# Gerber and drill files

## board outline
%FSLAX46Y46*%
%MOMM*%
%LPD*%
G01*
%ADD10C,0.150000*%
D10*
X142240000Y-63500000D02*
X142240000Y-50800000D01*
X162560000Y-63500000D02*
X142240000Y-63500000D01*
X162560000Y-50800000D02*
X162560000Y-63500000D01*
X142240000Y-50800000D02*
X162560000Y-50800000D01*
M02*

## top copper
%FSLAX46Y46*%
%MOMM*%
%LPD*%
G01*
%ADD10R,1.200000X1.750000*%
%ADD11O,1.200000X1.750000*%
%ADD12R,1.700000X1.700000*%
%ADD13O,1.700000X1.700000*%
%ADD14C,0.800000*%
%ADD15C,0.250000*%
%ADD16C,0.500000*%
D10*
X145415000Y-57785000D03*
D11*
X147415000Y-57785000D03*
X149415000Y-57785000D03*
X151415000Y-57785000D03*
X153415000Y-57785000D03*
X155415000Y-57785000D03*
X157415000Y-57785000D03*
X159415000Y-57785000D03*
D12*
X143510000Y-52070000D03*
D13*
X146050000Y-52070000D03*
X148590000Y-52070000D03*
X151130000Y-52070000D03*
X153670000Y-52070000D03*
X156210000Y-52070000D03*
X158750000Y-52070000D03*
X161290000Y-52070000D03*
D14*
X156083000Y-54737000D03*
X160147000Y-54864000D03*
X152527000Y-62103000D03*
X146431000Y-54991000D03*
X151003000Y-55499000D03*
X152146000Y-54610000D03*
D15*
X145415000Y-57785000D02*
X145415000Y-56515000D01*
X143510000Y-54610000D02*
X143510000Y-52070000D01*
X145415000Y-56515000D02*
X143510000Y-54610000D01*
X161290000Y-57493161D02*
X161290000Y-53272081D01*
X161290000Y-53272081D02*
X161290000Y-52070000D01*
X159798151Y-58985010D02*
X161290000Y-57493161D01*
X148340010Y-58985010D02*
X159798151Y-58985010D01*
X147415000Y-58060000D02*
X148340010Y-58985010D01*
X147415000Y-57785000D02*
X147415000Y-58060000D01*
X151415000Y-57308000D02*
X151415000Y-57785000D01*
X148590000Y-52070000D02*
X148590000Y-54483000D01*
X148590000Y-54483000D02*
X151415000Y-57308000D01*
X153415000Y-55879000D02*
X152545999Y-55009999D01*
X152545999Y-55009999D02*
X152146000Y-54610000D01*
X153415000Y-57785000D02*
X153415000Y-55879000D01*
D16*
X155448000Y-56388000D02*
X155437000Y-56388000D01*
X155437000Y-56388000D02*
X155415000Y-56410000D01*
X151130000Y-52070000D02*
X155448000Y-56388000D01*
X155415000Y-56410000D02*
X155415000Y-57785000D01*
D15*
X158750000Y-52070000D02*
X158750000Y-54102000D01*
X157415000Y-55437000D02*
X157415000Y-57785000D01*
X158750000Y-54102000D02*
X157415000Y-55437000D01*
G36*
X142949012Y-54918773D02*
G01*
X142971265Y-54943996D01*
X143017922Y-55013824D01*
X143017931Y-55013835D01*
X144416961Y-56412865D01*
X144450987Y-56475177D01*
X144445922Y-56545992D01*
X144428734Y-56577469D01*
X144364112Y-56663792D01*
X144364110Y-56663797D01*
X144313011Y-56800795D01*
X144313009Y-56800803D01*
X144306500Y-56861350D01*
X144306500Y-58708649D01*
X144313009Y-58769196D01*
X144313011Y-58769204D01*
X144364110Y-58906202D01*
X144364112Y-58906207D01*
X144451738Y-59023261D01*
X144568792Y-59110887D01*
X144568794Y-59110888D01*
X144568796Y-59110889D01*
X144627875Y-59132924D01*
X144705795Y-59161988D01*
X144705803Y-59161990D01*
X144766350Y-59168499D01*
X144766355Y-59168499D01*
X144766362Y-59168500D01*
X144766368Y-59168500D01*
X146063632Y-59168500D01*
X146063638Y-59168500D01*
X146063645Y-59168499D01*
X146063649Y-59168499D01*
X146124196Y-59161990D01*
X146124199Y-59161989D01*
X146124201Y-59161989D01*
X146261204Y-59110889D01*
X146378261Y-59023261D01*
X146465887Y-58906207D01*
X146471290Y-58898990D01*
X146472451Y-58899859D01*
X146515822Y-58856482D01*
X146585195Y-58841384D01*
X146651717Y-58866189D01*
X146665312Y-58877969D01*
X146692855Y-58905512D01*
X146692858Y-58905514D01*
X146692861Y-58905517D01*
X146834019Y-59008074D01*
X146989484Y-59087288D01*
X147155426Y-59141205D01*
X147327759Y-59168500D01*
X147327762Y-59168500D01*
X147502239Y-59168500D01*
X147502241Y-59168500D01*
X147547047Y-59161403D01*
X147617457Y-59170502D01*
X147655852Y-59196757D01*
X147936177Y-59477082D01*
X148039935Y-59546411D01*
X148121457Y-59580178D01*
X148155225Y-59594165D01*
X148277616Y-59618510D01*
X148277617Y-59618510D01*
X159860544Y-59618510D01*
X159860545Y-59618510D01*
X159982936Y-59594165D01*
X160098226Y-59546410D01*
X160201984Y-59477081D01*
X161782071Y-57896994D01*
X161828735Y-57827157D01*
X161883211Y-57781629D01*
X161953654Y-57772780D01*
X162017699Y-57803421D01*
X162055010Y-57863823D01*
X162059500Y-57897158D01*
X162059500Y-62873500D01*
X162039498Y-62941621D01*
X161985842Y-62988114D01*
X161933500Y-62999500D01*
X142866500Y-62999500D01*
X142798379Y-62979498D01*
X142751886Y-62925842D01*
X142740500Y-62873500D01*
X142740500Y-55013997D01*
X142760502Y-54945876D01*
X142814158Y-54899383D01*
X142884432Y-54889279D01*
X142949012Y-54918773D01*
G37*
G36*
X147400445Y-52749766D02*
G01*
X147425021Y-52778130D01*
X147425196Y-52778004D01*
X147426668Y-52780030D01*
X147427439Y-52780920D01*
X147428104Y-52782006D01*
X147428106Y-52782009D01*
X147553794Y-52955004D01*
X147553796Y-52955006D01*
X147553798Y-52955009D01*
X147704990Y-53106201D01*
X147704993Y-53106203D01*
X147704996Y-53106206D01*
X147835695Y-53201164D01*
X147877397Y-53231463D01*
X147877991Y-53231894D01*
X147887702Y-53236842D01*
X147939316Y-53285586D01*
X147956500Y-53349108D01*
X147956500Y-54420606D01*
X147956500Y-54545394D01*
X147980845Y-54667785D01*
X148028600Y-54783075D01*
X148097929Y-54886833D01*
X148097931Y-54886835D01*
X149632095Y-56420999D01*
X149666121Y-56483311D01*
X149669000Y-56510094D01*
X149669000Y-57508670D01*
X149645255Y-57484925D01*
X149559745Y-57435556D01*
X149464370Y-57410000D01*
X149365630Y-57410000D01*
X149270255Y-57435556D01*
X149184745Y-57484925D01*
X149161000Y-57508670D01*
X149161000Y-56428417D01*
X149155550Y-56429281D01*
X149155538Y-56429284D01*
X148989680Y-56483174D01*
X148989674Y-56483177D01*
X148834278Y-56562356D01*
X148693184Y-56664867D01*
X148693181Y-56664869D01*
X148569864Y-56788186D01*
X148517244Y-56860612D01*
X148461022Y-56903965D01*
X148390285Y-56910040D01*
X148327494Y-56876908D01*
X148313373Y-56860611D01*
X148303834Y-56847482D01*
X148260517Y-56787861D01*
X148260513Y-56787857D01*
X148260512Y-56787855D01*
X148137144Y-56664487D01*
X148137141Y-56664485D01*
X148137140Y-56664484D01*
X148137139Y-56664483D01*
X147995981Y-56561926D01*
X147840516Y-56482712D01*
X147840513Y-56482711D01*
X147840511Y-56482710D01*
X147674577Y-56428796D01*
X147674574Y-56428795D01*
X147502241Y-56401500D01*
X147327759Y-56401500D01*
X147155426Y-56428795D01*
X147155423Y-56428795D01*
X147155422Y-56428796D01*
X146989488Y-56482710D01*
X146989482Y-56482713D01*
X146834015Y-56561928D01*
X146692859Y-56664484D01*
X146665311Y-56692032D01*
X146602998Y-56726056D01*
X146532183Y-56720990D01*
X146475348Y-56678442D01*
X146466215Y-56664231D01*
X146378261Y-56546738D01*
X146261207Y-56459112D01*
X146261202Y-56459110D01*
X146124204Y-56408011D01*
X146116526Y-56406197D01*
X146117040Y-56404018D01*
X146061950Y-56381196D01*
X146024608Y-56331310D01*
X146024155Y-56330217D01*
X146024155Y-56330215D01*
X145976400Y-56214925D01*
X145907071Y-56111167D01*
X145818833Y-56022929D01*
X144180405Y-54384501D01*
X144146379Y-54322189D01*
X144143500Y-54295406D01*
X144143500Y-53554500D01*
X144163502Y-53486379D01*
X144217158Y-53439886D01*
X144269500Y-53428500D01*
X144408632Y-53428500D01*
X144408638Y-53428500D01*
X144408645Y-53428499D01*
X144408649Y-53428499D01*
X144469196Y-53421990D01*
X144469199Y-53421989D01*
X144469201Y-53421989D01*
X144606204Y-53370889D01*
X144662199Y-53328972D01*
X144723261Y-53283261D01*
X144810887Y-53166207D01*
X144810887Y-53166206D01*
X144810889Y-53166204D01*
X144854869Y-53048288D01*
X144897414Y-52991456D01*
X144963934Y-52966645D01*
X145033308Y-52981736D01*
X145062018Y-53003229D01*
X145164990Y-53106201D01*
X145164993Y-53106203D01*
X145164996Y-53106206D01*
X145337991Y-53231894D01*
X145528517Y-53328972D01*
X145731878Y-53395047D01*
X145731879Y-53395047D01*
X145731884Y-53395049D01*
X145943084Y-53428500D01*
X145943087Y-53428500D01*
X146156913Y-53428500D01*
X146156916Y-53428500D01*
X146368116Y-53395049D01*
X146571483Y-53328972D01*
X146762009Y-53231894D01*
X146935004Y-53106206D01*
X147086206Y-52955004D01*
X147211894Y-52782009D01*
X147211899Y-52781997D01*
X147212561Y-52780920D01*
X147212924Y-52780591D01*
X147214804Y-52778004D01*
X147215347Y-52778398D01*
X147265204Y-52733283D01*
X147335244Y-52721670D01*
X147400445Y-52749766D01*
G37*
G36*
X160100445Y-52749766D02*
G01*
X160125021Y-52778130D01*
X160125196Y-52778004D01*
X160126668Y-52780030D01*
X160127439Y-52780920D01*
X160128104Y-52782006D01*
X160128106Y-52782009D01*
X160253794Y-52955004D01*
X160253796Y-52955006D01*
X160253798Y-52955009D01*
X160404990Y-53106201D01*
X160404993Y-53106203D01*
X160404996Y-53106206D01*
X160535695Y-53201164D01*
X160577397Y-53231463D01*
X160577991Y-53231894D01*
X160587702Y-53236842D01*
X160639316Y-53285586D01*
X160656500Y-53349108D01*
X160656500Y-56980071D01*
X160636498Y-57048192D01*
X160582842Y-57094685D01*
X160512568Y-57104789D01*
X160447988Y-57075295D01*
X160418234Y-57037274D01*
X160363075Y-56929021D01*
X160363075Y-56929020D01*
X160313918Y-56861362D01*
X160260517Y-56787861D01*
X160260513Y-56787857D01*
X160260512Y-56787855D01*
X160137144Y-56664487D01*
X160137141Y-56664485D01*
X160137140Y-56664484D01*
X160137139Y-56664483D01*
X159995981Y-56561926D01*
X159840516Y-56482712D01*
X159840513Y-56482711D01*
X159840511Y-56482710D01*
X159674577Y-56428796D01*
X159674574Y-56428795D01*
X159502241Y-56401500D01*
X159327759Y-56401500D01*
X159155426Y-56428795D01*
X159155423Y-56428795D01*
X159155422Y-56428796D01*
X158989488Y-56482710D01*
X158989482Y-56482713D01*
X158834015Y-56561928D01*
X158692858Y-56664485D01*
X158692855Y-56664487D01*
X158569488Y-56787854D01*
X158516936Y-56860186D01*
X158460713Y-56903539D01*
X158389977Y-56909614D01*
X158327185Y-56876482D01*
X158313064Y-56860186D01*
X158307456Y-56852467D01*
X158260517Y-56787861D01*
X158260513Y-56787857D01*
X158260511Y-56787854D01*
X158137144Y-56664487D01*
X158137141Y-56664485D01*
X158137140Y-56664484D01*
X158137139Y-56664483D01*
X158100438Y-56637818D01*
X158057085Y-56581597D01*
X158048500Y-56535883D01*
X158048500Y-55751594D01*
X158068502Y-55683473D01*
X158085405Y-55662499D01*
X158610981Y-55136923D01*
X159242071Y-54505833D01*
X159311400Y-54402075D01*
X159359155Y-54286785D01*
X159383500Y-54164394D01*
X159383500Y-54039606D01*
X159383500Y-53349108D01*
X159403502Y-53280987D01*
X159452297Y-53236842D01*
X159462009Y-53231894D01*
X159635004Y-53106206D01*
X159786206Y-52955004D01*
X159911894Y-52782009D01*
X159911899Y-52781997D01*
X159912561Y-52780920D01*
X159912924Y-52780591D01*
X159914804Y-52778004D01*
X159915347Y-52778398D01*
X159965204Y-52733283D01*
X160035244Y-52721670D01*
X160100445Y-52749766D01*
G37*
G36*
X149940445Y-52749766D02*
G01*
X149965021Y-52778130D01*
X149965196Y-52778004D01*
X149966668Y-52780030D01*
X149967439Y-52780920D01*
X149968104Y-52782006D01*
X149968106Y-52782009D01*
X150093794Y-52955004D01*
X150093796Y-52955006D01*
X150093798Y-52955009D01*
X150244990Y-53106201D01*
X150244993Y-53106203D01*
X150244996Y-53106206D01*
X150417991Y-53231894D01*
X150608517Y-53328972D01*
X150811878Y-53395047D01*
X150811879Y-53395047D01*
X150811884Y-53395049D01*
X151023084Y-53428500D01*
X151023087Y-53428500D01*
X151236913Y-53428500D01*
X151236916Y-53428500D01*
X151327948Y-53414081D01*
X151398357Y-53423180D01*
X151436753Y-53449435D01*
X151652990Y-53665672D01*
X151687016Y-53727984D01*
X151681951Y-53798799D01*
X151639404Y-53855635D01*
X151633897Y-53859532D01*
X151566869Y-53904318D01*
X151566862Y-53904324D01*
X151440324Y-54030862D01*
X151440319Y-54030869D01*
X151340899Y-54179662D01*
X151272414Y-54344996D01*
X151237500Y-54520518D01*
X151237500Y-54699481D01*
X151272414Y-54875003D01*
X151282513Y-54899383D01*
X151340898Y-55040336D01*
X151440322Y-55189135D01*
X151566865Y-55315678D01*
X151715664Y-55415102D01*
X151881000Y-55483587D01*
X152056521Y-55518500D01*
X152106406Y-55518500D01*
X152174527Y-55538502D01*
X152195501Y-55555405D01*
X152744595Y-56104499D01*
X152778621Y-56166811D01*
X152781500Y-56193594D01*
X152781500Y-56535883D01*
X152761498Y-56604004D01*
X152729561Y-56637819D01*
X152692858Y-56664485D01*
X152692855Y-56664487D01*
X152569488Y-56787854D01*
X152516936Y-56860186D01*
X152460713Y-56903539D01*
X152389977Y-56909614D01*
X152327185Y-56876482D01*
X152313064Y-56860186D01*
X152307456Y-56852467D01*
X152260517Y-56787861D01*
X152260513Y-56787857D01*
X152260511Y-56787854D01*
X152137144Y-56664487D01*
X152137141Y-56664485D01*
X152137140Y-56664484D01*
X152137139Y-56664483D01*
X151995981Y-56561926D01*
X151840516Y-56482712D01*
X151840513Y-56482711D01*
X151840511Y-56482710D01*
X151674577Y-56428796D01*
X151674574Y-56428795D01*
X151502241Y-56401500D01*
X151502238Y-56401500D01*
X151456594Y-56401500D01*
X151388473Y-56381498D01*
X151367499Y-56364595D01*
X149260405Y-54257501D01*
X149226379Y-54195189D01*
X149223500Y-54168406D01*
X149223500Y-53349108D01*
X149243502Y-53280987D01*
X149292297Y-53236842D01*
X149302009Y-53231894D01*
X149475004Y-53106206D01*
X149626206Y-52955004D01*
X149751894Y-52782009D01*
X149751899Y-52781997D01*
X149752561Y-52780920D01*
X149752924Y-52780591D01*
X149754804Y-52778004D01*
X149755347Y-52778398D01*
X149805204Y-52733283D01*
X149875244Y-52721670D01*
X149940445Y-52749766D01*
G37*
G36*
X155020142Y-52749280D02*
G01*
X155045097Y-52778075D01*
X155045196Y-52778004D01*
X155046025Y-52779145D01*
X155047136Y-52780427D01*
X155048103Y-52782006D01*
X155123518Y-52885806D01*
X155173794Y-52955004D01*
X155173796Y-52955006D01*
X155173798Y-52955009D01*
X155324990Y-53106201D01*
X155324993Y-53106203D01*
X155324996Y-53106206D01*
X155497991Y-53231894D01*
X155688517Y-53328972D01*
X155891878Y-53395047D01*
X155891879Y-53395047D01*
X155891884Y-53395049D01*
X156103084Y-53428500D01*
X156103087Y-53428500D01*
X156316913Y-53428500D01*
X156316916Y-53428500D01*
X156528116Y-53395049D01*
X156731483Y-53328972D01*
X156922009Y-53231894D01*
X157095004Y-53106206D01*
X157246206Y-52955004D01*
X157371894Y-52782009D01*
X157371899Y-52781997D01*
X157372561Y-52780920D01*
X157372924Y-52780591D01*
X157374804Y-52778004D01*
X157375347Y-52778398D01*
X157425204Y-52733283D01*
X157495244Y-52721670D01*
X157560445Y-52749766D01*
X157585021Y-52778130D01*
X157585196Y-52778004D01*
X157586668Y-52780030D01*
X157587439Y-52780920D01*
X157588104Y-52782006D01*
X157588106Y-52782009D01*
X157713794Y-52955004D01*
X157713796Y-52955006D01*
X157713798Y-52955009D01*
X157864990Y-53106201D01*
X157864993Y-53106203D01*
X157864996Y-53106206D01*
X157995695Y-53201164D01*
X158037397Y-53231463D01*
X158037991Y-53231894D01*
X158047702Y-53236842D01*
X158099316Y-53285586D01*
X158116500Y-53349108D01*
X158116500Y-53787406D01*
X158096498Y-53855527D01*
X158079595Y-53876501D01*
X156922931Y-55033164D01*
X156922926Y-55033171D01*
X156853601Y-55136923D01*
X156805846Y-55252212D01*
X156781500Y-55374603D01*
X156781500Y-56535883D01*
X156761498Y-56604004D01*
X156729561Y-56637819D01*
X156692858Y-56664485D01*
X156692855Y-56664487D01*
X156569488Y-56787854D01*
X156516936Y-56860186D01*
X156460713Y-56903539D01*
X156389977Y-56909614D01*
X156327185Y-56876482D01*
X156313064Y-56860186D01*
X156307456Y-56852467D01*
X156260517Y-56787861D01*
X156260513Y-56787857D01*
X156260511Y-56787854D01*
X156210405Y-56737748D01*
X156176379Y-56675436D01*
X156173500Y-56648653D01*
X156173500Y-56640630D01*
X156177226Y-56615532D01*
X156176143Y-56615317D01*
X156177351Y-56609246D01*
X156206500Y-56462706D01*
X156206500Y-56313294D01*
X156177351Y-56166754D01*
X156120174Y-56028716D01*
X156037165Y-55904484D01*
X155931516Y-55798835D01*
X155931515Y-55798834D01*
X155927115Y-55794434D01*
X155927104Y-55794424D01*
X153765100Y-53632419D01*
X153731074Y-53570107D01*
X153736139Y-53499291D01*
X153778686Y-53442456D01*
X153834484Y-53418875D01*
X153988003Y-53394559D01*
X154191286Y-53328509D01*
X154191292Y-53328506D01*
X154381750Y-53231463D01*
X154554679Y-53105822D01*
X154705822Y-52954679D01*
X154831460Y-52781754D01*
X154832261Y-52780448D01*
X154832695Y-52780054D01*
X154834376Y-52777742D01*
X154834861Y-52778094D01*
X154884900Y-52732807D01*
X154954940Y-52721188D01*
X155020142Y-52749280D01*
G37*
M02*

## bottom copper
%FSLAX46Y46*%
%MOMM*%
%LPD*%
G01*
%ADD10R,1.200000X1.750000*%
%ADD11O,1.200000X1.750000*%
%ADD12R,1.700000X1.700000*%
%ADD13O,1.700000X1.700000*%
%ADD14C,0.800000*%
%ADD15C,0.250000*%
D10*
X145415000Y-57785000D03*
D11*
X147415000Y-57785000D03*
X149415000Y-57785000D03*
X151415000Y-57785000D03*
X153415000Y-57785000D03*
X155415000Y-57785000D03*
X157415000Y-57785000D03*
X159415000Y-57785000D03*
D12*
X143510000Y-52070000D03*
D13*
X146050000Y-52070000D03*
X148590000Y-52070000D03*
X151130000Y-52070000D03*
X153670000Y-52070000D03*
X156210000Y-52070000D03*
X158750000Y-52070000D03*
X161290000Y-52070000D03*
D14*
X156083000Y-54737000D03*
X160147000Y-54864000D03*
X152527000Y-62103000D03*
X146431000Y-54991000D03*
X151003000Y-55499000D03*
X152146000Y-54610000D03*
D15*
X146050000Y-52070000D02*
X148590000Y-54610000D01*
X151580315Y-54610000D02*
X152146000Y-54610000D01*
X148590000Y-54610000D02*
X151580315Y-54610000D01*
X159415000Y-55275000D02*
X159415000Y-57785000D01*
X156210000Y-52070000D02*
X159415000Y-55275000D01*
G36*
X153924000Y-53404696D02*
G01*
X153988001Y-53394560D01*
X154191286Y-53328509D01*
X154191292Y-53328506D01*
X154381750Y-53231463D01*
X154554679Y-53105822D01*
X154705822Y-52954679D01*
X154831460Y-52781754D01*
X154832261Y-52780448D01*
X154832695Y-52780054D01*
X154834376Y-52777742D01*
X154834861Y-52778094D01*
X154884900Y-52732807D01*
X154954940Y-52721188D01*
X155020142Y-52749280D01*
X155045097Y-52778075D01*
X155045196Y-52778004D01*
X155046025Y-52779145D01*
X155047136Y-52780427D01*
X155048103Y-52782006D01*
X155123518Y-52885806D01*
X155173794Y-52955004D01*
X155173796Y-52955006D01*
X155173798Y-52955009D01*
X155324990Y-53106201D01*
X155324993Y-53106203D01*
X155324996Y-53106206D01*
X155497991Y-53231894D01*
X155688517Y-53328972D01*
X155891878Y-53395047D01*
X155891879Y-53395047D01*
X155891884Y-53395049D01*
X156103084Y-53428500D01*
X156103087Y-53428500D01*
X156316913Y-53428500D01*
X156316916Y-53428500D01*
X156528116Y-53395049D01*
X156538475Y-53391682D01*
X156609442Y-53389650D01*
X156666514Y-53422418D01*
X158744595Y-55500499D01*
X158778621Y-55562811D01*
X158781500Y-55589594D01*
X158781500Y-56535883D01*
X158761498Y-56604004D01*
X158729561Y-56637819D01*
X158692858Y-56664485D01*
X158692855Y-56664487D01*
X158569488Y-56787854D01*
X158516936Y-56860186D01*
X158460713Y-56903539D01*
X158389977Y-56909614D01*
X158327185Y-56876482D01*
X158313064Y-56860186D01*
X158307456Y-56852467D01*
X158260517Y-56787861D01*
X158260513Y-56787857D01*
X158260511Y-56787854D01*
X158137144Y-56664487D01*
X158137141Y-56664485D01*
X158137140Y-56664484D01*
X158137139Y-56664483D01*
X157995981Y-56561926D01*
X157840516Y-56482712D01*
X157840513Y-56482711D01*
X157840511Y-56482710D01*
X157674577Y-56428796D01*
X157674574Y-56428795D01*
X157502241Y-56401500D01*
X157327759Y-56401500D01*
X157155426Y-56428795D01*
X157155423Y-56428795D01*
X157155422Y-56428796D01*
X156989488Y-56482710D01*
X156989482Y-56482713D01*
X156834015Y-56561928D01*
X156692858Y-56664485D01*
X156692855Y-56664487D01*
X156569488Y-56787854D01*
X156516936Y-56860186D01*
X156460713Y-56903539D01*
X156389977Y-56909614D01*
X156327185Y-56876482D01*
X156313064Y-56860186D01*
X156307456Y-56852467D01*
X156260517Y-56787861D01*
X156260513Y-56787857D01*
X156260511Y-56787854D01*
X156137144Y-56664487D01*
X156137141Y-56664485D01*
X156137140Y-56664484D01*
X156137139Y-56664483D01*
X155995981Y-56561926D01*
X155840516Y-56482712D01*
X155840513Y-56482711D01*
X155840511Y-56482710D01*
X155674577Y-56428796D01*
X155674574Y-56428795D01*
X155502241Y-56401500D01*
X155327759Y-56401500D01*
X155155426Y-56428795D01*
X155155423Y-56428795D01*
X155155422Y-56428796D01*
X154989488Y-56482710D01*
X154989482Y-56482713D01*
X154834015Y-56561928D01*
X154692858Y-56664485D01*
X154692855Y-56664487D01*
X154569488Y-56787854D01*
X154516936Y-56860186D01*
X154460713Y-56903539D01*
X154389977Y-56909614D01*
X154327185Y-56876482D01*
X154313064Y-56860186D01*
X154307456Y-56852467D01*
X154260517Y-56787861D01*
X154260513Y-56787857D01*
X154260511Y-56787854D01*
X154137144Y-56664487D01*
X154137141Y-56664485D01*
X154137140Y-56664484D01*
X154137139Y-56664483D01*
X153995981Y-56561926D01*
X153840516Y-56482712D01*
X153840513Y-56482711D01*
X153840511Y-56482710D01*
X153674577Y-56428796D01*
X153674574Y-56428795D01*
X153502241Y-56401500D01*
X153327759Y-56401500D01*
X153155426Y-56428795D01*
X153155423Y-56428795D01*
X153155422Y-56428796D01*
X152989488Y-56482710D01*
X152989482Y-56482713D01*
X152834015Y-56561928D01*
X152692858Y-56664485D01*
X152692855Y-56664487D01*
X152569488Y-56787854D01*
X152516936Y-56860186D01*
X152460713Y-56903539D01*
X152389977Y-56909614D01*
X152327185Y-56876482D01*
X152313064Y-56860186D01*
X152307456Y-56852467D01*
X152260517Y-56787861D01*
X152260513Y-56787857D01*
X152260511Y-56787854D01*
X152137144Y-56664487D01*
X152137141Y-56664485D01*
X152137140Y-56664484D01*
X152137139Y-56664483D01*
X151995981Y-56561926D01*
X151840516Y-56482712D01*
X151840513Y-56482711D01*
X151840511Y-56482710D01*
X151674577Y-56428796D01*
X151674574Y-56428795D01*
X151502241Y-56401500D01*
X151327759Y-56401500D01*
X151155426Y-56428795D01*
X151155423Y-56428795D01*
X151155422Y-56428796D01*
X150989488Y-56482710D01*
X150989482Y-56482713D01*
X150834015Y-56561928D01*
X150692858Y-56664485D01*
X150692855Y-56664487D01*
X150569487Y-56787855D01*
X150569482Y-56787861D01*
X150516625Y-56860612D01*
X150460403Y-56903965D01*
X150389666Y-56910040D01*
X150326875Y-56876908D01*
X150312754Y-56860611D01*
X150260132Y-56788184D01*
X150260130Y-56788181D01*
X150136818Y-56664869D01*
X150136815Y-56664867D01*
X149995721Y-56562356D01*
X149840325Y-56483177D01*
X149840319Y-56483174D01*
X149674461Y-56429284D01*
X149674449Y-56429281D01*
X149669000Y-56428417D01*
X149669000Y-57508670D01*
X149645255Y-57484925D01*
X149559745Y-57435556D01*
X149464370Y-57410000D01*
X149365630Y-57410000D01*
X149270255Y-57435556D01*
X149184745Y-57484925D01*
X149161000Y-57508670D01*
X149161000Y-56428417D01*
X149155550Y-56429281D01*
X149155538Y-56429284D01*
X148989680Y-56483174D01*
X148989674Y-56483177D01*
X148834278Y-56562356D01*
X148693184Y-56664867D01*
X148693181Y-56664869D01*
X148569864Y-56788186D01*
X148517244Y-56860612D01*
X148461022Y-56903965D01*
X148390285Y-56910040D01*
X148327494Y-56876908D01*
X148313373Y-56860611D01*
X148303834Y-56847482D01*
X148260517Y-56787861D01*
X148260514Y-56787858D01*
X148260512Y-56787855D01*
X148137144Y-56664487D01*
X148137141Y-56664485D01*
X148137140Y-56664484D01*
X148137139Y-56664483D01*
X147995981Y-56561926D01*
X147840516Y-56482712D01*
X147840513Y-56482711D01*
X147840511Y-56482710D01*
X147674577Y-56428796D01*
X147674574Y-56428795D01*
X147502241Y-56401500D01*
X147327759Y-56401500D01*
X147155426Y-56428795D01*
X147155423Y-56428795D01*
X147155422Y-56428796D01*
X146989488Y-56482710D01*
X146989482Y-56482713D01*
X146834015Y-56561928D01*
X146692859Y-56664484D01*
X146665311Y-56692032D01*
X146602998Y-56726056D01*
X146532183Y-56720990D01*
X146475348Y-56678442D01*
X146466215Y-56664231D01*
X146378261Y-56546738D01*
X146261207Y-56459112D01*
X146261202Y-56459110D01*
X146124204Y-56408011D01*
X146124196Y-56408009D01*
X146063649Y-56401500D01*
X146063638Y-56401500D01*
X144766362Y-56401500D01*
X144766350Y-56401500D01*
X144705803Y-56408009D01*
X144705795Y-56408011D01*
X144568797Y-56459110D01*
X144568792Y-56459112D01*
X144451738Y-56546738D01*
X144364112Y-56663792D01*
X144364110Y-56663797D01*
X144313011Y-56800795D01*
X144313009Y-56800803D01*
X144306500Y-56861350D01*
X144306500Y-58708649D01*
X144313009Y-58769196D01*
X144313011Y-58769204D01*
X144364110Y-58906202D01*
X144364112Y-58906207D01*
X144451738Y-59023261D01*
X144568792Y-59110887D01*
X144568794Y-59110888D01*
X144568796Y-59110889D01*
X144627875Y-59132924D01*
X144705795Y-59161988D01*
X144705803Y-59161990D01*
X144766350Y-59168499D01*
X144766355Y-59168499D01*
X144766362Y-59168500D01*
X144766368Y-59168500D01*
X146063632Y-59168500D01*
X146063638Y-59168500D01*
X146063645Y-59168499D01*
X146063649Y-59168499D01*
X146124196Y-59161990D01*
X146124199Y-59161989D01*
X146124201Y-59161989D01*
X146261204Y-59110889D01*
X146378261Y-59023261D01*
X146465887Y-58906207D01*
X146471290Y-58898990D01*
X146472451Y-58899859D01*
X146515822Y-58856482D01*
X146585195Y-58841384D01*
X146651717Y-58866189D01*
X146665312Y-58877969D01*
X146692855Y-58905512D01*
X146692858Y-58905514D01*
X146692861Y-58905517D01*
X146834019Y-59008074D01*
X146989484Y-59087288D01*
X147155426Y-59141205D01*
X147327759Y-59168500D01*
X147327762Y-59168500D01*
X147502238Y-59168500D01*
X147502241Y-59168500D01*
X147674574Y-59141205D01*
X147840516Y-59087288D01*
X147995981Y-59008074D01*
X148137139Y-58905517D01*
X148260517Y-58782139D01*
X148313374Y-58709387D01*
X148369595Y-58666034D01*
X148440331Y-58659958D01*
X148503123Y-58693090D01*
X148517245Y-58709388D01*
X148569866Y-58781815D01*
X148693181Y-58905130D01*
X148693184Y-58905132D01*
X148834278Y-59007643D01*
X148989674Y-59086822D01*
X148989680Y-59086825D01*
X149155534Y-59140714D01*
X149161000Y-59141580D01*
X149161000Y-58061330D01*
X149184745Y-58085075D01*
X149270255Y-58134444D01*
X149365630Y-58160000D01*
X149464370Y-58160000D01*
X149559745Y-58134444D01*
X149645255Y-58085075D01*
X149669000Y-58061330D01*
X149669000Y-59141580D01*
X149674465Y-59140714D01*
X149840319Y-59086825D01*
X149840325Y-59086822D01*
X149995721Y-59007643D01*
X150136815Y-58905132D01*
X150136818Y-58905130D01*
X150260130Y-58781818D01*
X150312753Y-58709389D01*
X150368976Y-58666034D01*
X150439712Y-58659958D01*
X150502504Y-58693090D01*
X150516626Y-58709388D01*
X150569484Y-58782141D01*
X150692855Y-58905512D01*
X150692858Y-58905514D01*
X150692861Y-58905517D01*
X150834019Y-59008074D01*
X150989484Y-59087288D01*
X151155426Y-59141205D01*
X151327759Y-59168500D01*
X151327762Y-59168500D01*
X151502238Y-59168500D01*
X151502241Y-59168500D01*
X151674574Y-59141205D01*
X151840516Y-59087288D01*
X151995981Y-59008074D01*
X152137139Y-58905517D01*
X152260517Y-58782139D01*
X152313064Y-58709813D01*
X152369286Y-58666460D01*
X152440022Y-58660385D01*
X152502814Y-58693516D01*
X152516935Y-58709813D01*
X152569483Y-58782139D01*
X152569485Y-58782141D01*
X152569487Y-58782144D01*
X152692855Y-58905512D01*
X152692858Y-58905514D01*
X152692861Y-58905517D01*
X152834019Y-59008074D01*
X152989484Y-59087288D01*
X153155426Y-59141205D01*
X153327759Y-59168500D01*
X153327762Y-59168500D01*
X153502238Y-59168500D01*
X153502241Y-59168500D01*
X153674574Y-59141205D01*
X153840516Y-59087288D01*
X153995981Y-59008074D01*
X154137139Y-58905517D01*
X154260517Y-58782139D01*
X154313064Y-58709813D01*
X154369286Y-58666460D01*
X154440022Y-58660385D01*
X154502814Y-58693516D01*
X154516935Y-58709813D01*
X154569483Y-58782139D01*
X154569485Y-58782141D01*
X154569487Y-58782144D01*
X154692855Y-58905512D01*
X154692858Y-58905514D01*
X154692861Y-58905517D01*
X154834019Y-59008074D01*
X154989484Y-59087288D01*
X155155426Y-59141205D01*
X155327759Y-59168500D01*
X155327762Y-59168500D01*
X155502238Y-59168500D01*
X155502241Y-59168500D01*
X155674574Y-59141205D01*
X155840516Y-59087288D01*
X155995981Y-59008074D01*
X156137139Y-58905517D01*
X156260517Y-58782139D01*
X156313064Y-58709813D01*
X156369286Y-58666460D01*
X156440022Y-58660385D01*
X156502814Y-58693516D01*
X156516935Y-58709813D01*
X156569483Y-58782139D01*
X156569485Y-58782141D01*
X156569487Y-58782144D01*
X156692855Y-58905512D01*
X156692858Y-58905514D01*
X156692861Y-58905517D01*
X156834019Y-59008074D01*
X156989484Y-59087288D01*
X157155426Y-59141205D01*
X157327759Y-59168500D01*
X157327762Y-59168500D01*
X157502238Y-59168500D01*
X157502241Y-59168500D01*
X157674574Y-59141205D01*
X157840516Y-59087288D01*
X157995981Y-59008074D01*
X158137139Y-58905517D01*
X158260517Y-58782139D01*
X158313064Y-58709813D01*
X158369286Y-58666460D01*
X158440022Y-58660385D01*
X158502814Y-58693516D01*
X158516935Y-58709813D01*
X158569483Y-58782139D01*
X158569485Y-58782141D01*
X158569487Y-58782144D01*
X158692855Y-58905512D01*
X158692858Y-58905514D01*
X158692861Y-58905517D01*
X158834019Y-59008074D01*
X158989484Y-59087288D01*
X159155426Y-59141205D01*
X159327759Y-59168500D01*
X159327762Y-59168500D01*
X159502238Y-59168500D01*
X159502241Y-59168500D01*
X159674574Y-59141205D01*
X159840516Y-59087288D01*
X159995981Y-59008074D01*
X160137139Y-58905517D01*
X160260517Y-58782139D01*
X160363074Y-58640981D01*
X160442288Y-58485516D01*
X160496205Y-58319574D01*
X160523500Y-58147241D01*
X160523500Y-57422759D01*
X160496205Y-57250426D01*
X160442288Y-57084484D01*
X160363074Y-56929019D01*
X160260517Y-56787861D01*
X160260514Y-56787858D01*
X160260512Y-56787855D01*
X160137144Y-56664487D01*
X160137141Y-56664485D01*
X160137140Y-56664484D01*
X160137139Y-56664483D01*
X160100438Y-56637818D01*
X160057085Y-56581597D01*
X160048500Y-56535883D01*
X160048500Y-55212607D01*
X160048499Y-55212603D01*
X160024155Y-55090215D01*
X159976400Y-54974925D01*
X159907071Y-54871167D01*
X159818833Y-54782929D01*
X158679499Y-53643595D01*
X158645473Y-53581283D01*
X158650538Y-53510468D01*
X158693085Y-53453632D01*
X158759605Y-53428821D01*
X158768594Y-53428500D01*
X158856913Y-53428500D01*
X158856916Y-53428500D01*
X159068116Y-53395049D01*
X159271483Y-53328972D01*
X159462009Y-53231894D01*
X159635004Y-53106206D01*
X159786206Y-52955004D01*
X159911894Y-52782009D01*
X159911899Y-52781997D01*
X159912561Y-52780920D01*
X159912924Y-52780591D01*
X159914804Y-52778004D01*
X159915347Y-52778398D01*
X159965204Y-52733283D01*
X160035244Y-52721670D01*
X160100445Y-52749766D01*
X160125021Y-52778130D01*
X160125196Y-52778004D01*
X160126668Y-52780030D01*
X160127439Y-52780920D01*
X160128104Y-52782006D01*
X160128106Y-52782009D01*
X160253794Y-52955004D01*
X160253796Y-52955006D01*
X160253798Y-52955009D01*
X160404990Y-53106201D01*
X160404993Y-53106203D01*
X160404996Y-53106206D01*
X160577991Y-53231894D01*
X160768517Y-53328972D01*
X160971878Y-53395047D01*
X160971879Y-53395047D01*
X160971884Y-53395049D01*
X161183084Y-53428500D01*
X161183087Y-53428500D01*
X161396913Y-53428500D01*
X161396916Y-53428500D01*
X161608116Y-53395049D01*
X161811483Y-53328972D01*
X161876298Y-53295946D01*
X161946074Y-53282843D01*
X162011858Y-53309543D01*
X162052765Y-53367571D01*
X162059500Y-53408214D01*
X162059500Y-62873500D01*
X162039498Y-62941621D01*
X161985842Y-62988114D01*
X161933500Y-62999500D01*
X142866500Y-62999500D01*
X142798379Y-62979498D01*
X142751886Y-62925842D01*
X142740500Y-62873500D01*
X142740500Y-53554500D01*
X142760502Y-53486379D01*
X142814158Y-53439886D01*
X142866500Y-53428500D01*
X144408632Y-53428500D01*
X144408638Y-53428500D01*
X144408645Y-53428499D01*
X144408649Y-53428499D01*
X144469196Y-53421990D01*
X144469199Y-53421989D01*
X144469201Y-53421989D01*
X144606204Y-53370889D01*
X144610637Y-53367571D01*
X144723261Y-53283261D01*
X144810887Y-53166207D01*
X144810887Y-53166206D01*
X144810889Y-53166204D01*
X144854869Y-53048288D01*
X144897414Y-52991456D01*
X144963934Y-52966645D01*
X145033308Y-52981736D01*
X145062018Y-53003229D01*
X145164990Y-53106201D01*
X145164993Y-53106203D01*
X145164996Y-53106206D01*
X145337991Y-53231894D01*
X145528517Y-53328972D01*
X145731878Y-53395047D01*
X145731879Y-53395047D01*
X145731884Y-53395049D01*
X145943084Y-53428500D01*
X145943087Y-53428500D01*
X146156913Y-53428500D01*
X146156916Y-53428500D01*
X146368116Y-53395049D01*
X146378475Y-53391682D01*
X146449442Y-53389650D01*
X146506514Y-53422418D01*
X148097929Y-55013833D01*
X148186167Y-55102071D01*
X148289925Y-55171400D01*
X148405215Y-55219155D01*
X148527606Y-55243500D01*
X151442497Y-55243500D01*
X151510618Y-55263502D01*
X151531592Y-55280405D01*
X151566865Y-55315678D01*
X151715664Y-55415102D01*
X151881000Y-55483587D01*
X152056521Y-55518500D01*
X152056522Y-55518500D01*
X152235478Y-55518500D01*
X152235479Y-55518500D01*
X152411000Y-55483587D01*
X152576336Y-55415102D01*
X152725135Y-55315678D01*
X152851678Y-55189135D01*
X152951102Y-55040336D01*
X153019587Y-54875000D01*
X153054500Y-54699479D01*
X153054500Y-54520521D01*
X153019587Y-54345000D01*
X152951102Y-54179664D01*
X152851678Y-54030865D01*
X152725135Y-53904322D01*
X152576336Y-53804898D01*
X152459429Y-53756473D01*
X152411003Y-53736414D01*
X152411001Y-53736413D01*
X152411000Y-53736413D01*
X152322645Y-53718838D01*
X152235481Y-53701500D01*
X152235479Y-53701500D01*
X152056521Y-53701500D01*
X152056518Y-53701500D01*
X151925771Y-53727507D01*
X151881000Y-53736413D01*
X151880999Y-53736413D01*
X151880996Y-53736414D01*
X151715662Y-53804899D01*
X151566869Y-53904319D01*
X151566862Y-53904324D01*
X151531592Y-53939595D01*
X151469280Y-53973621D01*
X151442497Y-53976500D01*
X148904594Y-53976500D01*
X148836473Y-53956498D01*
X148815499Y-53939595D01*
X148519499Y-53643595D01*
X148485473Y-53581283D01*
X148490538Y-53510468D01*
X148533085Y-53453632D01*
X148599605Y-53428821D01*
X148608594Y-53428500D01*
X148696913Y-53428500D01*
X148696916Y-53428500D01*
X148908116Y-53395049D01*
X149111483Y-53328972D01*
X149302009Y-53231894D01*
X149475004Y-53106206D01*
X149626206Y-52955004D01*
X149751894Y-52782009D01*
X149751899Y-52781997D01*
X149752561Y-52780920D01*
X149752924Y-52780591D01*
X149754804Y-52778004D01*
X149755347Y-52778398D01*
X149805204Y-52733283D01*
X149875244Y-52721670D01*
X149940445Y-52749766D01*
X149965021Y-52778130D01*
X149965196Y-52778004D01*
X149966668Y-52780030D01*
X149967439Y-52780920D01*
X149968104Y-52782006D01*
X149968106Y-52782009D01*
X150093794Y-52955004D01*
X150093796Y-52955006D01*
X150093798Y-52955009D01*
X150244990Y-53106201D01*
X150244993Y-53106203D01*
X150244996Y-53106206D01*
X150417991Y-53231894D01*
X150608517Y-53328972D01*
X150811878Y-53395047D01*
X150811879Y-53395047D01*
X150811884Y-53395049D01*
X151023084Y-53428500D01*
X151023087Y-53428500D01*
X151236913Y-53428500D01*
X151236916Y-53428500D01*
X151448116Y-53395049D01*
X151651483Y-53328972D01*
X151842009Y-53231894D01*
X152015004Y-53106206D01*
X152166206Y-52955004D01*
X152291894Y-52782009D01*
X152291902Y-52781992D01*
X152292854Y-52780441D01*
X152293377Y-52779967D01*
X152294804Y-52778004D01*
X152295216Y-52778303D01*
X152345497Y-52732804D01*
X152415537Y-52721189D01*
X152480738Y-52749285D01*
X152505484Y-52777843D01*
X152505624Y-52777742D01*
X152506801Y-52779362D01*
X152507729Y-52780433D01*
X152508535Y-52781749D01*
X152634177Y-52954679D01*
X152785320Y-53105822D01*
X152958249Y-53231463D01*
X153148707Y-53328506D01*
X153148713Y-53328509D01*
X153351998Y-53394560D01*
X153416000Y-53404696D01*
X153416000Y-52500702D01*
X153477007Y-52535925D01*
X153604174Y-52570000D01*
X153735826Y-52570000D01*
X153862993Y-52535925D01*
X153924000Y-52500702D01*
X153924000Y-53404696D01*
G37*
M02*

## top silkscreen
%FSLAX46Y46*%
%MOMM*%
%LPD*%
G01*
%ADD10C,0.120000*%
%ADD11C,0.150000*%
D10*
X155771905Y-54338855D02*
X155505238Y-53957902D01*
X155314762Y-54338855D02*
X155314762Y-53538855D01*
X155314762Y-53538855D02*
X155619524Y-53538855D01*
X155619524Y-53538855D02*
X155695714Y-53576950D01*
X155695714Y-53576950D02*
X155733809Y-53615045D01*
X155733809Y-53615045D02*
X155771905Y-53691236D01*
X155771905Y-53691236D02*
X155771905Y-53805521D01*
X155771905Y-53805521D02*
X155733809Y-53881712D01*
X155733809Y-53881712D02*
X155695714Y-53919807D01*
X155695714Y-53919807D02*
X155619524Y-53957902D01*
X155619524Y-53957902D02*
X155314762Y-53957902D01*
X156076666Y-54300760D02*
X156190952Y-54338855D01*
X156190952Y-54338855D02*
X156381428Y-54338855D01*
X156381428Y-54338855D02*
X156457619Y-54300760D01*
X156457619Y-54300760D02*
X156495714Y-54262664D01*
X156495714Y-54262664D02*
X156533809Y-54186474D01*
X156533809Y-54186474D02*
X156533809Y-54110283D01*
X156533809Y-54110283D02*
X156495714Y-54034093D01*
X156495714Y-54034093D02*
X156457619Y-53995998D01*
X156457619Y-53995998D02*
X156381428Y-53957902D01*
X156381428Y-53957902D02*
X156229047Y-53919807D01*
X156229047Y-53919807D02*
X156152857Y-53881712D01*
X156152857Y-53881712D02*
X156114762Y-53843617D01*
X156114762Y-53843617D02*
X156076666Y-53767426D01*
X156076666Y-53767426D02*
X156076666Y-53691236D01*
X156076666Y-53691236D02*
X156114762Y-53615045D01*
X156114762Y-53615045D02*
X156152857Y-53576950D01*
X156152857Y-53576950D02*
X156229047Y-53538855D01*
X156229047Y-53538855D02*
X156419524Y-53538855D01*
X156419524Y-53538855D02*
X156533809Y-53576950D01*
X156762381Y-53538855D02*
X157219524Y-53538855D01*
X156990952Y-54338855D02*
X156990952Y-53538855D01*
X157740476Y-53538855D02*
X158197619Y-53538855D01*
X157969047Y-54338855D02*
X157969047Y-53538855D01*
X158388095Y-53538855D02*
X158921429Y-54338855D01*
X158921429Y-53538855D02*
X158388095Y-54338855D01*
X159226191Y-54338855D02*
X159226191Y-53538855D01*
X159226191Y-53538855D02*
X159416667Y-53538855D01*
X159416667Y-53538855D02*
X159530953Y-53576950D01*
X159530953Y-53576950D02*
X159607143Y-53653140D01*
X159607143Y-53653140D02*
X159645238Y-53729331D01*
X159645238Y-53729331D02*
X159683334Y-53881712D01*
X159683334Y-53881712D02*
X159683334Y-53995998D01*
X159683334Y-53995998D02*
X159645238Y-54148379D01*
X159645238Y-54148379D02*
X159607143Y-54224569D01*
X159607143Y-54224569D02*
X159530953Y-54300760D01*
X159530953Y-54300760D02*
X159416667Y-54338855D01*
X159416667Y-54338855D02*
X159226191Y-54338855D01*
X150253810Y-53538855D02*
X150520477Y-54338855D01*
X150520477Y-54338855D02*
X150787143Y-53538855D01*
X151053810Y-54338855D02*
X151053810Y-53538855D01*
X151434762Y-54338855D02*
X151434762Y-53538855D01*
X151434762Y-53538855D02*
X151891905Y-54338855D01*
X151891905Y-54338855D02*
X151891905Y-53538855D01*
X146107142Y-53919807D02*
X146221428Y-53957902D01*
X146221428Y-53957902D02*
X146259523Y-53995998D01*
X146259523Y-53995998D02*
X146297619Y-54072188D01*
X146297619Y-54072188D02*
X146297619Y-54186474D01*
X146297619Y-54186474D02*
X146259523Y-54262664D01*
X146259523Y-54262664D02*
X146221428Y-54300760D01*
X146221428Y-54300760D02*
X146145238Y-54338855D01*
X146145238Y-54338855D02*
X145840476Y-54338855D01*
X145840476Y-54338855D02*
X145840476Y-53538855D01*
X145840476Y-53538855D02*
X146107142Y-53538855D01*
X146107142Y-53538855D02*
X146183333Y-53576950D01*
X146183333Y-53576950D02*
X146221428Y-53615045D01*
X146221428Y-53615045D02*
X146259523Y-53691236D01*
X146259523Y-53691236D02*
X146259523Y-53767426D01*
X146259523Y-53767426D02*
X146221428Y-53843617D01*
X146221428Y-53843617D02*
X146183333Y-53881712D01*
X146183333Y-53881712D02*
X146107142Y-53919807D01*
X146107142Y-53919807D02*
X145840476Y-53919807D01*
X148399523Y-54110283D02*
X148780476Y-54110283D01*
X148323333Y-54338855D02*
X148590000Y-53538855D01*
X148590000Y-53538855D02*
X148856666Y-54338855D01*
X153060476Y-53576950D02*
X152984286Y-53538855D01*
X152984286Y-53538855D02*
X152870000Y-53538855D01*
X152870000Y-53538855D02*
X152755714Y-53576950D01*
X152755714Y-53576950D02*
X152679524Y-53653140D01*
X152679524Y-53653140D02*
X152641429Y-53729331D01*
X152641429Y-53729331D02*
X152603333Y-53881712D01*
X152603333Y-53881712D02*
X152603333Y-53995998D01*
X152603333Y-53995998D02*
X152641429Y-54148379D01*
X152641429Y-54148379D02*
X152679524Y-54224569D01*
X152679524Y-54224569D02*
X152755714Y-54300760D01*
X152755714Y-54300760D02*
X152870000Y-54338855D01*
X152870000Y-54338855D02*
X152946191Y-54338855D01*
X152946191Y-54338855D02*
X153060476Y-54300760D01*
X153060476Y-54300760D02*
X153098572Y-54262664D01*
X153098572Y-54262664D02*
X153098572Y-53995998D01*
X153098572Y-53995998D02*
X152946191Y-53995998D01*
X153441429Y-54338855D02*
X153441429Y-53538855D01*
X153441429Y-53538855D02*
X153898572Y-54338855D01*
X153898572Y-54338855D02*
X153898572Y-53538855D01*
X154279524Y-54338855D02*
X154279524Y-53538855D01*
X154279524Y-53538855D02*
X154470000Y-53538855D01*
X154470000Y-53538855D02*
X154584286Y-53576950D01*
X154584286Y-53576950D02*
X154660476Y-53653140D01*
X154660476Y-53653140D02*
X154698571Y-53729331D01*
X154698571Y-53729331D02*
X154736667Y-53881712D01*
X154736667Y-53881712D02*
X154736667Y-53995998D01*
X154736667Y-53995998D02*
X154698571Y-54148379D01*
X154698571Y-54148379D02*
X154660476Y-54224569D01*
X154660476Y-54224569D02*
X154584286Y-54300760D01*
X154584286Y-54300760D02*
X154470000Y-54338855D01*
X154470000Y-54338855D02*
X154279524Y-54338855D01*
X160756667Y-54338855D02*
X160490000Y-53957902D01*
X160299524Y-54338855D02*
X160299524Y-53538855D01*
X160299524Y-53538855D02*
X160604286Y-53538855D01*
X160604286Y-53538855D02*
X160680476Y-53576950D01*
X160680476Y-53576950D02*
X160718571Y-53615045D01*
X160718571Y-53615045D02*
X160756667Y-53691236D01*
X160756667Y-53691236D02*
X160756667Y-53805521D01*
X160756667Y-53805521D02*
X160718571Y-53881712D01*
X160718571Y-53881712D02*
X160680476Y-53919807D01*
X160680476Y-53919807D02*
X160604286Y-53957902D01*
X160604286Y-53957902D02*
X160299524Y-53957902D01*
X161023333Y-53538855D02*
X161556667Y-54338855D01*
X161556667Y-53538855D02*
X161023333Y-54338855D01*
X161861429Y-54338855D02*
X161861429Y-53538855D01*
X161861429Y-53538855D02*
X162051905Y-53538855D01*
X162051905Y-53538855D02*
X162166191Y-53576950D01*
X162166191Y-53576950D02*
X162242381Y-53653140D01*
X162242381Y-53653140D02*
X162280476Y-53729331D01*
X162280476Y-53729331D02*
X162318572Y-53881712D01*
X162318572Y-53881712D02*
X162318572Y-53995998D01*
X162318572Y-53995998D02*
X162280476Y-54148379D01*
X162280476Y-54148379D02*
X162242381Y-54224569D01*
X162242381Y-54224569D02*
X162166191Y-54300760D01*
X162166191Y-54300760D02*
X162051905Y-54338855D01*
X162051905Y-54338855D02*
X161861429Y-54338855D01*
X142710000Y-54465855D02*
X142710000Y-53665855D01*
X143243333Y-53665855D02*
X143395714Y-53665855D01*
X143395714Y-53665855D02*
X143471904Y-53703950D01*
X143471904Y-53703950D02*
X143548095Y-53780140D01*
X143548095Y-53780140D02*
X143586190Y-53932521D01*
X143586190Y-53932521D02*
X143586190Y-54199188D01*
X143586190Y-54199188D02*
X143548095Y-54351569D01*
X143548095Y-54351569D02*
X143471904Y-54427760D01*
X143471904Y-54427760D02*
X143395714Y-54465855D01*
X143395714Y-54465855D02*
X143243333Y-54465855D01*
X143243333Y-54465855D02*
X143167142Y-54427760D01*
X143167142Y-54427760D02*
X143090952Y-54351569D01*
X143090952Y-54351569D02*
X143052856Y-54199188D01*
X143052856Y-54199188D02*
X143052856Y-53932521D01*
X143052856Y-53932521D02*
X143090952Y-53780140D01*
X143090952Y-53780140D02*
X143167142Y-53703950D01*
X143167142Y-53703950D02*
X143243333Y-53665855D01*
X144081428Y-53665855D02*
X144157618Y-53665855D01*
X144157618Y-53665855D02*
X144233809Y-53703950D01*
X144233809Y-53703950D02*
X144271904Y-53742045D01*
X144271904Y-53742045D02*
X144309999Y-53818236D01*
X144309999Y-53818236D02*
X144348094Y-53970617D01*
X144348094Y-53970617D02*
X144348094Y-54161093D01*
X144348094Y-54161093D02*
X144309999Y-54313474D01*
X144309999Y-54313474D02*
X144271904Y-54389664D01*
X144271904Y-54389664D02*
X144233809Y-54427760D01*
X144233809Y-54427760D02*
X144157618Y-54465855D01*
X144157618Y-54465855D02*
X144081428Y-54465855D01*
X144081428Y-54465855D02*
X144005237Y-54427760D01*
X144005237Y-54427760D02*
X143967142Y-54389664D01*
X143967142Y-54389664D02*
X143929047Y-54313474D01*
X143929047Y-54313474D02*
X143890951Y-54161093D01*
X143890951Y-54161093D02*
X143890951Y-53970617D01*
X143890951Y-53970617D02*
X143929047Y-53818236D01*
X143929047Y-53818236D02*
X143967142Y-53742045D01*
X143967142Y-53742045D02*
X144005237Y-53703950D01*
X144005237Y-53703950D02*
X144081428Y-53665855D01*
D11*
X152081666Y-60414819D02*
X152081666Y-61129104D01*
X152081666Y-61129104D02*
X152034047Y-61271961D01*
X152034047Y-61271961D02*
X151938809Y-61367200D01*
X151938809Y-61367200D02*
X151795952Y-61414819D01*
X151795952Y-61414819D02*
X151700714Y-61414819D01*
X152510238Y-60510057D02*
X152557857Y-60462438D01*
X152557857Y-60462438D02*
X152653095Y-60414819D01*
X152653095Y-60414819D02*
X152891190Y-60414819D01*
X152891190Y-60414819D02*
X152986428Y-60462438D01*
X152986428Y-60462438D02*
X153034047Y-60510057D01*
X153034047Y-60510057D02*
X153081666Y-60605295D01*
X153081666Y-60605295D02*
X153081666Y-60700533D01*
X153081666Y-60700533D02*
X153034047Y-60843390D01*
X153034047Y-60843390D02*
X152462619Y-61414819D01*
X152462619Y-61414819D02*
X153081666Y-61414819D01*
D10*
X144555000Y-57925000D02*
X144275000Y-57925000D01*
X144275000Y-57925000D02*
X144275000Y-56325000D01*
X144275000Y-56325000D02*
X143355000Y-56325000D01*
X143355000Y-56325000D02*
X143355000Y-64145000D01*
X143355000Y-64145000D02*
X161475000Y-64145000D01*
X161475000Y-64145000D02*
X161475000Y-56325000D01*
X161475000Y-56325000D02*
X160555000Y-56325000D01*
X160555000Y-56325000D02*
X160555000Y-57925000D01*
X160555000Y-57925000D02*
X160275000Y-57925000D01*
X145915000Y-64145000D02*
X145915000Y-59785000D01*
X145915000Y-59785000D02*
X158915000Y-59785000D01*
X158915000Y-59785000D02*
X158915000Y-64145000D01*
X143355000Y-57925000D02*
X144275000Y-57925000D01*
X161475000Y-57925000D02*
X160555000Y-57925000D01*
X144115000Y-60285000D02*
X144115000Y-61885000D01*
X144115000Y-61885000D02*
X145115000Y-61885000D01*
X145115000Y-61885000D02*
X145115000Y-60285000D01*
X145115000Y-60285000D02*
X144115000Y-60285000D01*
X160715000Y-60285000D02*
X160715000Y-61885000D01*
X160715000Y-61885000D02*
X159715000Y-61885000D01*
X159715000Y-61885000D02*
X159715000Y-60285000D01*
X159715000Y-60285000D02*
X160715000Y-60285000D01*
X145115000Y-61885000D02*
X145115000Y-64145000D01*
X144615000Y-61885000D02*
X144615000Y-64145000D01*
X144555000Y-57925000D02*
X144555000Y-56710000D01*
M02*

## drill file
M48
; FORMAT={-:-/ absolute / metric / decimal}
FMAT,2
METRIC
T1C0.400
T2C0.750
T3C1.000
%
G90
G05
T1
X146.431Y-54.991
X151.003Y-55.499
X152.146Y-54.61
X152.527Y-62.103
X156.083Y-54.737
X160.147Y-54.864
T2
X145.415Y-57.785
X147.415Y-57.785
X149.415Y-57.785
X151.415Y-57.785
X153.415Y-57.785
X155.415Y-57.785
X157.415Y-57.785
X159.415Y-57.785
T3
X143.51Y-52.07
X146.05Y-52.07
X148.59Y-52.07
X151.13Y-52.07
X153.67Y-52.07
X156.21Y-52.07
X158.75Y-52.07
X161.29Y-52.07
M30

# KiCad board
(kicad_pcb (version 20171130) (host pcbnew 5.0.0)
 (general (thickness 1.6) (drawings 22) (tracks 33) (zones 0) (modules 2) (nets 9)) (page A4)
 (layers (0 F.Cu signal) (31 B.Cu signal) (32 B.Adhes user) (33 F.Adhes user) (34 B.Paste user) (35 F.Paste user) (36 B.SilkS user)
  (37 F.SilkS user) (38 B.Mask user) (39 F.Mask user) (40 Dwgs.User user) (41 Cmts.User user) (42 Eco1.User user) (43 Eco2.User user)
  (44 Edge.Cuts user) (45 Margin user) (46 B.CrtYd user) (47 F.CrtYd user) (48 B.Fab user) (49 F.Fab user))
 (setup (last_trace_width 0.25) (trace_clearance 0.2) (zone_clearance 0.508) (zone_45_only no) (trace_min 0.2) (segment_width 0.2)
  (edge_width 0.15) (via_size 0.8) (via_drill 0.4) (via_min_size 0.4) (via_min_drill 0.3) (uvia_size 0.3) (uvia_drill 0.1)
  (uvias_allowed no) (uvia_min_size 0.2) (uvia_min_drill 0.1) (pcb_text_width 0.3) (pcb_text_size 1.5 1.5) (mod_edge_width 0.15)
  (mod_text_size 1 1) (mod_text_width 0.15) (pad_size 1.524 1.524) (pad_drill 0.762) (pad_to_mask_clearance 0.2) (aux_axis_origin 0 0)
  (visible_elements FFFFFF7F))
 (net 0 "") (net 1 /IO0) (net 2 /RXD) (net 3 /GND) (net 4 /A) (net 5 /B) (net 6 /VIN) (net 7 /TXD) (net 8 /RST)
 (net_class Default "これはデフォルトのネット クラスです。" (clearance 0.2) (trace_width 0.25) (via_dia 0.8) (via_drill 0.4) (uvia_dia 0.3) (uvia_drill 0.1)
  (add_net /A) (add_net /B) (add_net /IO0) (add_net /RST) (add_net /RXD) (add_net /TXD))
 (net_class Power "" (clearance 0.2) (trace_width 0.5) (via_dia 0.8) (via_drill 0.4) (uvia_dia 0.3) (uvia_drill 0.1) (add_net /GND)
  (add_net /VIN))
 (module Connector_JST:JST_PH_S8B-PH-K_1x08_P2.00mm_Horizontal (layer F.Cu) (at 145.415 57.785)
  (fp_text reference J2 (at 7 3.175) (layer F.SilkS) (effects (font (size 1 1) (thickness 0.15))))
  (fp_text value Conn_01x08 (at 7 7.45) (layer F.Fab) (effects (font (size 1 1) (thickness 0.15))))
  (fp_line (start -0.86 0.14) (end -1.14 0.14) (layer F.SilkS) (width 0.12))
  (fp_line (start -1.14 0.14) (end -1.14 -1.46) (layer F.SilkS) (width 0.12))
  (fp_line (start -1.14 -1.46) (end -2.06 -1.46) (layer F.SilkS) (width 0.12))
  (fp_line (start -2.06 -1.46) (end -2.06 6.36) (layer F.SilkS) (width 0.12))
  (fp_line (start -2.06 6.36) (end 16.06 6.36) (layer F.SilkS) (width 0.12))
  (fp_line (start 16.06 6.36) (end 16.06 -1.46) (layer F.SilkS) (width 0.12))
  (fp_line (start 16.06 -1.46) (end 15.14 -1.46) (layer F.SilkS) (width 0.12))
  (fp_line (start 15.14 -1.46) (end 15.14 0.14) (layer F.SilkS) (width 0.12))
  (fp_line (start 15.14 0.14) (end 14.86 0.14) (layer F.SilkS) (width 0.12))
  (fp_line (start 0.5 6.36) (end 0.5 2) (layer F.SilkS) (width 0.12))
  (fp_line (start 0.5 2) (end 13.5 2) (layer F.SilkS) (width 0.12))
  (fp_line (start 13.5 2) (end 13.5 6.36) (layer F.SilkS) (width 0.12))
  (fp_line (start -2.06 0.14) (end -1.14 0.14) (layer F.SilkS) (width 0.12))
  (fp_line (start 16.06 0.14) (end 15.14 0.14) (layer F.SilkS) (width 0.12))
  (fp_line (start -1.3 2.5) (end -1.3 4.1) (layer F.SilkS) (width 0.12))
  (fp_line (start -1.3 4.1) (end -0.3 4.1) (layer F.SilkS) (width 0.12))
  (fp_line (start -0.3 4.1) (end -0.3 2.5) (layer F.SilkS) (width 0.12))
  (fp_line (start -0.3 2.5) (end -1.3 2.5) (layer F.SilkS) (width 0.12))
  (fp_line (start 15.3 2.5) (end 15.3 4.1) (layer F.SilkS) (width 0.12))
  (fp_line (start 15.3 4.1) (end 14.3 4.1) (layer F.SilkS) (width 0.12))
  (fp_line (start 14.3 4.1) (end 14.3 2.5) (layer F.SilkS) (width 0.12))
  (fp_line (start 14.3 2.5) (end 15.3 2.5) (layer F.SilkS) (width 0.12))
  (fp_line (start -0.3 4.1) (end -0.3 6.36) (layer F.SilkS) (width 0.12))
  (fp_line (start -0.8 4.1) (end -0.8 6.36) (layer F.SilkS) (width 0.12))
  (fp_line (start -0.86 0.14) (end -0.86 -1.075) (layer F.SilkS) (width 0.12))
  (pad 1 thru_hole rect (at 0 0) (size 1.2 1.75) (drill 0.75) (layers *.Cu *.Mask) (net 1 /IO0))
  (pad 2 thru_hole oval (at 2 0) (size 1.2 1.75) (drill 0.75) (layers *.Cu *.Mask) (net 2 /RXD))
  (pad 3 thru_hole oval (at 4 0) (size 1.2 1.75) (drill 0.75) (layers *.Cu *.Mask) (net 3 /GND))
  (pad 4 thru_hole oval (at 6 0) (size 1.2 1.75) (drill 0.75) (layers *.Cu *.Mask) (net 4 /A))
  (pad 5 thru_hole oval (at 8 0) (size 1.2 1.75) (drill 0.75) (layers *.Cu *.Mask) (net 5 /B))
  (pad 6 thru_hole oval (at 10 0) (size 1.2 1.75) (drill 0.75) (layers *.Cu *.Mask) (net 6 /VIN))
  (pad 7 thru_hole oval (at 12 0) (size 1.2 1.75) (drill 0.75) (layers *.Cu *.Mask) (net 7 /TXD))
  (pad 8 thru_hole oval (at 14 0) (size 1.2 1.75) (drill 0.75) (layers *.Cu *.Mask) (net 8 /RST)))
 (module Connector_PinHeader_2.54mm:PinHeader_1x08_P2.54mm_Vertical (layer B.Cu) (at 143.51 52.07 270)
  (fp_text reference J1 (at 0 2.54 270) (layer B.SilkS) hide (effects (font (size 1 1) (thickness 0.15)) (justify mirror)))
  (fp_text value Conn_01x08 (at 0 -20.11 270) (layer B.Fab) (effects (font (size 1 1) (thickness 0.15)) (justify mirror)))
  (pad 1 thru_hole rect (at 0 0 270) (size 1.7 1.7) (drill 1) (layers *.Cu *.Mask) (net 1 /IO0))
  (pad 2 thru_hole oval (at 0 -2.54 270) (size 1.7 1.7) (drill 1) (layers *.Cu *.Mask) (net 5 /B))
  (pad 3 thru_hole oval (at 0 -5.08 270) (size 1.7 1.7) (drill 1) (layers *.Cu *.Mask) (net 4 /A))
  (pad 4 thru_hole oval (at 0 -7.62 270) (size 1.7 1.7) (drill 1) (layers *.Cu *.Mask) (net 6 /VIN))
  (pad 5 thru_hole oval (at 0 -10.16 270) (size 1.7 1.7) (drill 1) (layers *.Cu *.Mask) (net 3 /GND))
  (pad 6 thru_hole oval (at 0 -12.7 270) (size 1.7 1.7) (drill 1) (layers *.Cu *.Mask) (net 8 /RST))
  (pad 7 thru_hole oval (at 0 -15.24 270) (size 1.7 1.7) (drill 1) (layers *.Cu *.Mask) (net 7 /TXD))
  (pad 8 thru_hole oval (at 0 -17.78 270) (size 1.7 1.7) (drill 1) (layers *.Cu *.Mask) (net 2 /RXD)))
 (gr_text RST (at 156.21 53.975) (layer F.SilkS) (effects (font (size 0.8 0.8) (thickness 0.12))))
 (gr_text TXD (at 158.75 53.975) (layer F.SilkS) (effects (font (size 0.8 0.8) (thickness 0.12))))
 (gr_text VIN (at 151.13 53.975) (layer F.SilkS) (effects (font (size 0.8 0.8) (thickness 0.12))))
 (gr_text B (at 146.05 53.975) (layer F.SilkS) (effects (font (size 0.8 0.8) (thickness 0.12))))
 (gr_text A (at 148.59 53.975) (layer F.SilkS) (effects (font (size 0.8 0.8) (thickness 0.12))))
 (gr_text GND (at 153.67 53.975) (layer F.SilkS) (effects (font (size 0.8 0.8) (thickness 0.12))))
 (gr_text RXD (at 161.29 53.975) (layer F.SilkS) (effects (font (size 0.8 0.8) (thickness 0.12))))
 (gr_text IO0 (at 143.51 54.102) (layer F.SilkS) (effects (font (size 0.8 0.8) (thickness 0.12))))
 (gr_line (start 142.24 63.5) (end 142.24 50.8) (layer Edge.Cuts) (width 0.15))
 (gr_line (start 162.56 63.5) (end 142.24 63.5) (layer Edge.Cuts) (width 0.15))
 (gr_line (start 162.56 50.8) (end 162.56 63.5) (layer Edge.Cuts) (width 0.15))
 (gr_line (start 142.24 50.8) (end 162.56 50.8) (layer Edge.Cuts) (width 0.15))
 (segment (start 145.415 57.785) (end 145.415 56.515) (width 0.25) (layer F.Cu) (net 1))
 (segment (start 143.51 54.61) (end 143.51 52.07) (width 0.25) (layer F.Cu) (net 1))
 (segment (start 145.415 56.515) (end 143.51 54.61) (width 0.25) (layer F.Cu) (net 1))
 (segment (start 161.29 57.493161) (end 161.29 53.272081) (width 0.25) (layer F.Cu) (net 2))
 (segment (start 161.29 53.272081) (end 161.29 52.07) (width 0.25) (layer F.Cu) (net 2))
 (segment (start 159.798151 58.98501) (end 161.29 57.493161) (width 0.25) (layer F.Cu) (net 2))
 (segment (start 148.34001 58.98501) (end 159.798151 58.98501) (width 0.25) (layer F.Cu) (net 2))
 (segment (start 147.415 58.06) (end 148.34001 58.98501) (width 0.25) (layer F.Cu) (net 2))
 (segment (start 147.415 57.785) (end 147.415 58.06) (width 0.25) (layer F.Cu) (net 2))
 (via (at 156.083 54.737) (size 0.8) (drill 0.4) (layers F.Cu B.Cu) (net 3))
 (via (at 160.147 54.864) (size 0.8) (drill 0.4) (layers F.Cu B.Cu) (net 3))
 (via (at 152.527 62.103) (size 0.8) (drill 0.4) (layers F.Cu B.Cu) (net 3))
 (via (at 146.431 54.991) (size 0.8) (drill 0.4) (layers F.Cu B.Cu) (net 3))
 (via (at 151.003 55.499) (size 0.8) (drill 0.4) (layers F.Cu B.Cu) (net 3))
 (segment (start 151.415 57.308) (end 151.415 57.785) (width 0.25) (layer F.Cu) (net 4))
 (segment (start 148.59 52.07) (end 148.59 54.483) (width 0.25) (layer F.Cu) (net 4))
 (segment (start 148.59 54.483) (end 151.415 57.308) (width 0.25) (layer F.Cu) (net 4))
 (via (at 152.146 54.61) (size 0.8) (drill 0.4) (layers F.Cu B.Cu) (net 5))
 (segment (start 146.05 52.07) (end 148.59 54.61) (width 0.25) (layer B.Cu) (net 5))
 (segment (start 153.415 55.879) (end 152.545999 55.009999) (width 0.25) (layer F.Cu) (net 5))
 (segment (start 152.545999 55.009999) (end 152.146 54.61) (width 0.25) (layer F.Cu) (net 5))
 (segment (start 153.415 57.785) (end 153.415 55.879) (width 0.25) (layer F.Cu) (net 5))
 (segment (start 151.580315 54.61) (end 152.146 54.61) (width 0.25) (layer B.Cu) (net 5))
 (segment (start 148.59 54.61) (end 151.580315 54.61) (width 0.25) (layer B.Cu) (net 5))
 (segment (start 155.448 56.388) (end 155.437 56.388) (width 0.5) (layer F.Cu) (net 6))
 (segment (start 155.437 56.388) (end 155.415 56.41) (width 0.5) (layer F.Cu) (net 6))
 (segment (start 151.13 52.07) (end 155.448 56.388) (width 0.5) (layer F.Cu) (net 6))
 (segment (start 155.415 56.41) (end 155.415 57.785) (width 0.5) (layer F.Cu) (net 6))
 (segment (start 158.75 52.07) (end 158.75 54.102) (width 0.25) (layer F.Cu) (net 7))
 (segment (start 157.415 55.437) (end 157.415 57.785) (width 0.25) (layer F.Cu) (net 7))
 (segment (start 158.75 54.102) (end 157.415 55.437) (width 0.25) (layer F.Cu) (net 7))
 (segment (start 159.415 55.275) (end 159.415 57.785) (width 0.25) (layer B.Cu) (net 8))
 (segment (start 156.21 52.07) (end 159.415 55.275) (width 0.25) (layer B.Cu) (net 8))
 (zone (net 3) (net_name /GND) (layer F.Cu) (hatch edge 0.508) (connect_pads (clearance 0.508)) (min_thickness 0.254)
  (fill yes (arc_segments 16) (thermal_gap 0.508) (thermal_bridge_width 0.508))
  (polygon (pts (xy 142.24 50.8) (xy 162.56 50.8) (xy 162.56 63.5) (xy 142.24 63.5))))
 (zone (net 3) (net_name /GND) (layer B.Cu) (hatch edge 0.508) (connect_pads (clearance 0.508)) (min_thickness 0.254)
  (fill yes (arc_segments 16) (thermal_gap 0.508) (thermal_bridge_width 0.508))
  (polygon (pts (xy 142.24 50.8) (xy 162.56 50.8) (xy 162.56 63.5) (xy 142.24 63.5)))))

